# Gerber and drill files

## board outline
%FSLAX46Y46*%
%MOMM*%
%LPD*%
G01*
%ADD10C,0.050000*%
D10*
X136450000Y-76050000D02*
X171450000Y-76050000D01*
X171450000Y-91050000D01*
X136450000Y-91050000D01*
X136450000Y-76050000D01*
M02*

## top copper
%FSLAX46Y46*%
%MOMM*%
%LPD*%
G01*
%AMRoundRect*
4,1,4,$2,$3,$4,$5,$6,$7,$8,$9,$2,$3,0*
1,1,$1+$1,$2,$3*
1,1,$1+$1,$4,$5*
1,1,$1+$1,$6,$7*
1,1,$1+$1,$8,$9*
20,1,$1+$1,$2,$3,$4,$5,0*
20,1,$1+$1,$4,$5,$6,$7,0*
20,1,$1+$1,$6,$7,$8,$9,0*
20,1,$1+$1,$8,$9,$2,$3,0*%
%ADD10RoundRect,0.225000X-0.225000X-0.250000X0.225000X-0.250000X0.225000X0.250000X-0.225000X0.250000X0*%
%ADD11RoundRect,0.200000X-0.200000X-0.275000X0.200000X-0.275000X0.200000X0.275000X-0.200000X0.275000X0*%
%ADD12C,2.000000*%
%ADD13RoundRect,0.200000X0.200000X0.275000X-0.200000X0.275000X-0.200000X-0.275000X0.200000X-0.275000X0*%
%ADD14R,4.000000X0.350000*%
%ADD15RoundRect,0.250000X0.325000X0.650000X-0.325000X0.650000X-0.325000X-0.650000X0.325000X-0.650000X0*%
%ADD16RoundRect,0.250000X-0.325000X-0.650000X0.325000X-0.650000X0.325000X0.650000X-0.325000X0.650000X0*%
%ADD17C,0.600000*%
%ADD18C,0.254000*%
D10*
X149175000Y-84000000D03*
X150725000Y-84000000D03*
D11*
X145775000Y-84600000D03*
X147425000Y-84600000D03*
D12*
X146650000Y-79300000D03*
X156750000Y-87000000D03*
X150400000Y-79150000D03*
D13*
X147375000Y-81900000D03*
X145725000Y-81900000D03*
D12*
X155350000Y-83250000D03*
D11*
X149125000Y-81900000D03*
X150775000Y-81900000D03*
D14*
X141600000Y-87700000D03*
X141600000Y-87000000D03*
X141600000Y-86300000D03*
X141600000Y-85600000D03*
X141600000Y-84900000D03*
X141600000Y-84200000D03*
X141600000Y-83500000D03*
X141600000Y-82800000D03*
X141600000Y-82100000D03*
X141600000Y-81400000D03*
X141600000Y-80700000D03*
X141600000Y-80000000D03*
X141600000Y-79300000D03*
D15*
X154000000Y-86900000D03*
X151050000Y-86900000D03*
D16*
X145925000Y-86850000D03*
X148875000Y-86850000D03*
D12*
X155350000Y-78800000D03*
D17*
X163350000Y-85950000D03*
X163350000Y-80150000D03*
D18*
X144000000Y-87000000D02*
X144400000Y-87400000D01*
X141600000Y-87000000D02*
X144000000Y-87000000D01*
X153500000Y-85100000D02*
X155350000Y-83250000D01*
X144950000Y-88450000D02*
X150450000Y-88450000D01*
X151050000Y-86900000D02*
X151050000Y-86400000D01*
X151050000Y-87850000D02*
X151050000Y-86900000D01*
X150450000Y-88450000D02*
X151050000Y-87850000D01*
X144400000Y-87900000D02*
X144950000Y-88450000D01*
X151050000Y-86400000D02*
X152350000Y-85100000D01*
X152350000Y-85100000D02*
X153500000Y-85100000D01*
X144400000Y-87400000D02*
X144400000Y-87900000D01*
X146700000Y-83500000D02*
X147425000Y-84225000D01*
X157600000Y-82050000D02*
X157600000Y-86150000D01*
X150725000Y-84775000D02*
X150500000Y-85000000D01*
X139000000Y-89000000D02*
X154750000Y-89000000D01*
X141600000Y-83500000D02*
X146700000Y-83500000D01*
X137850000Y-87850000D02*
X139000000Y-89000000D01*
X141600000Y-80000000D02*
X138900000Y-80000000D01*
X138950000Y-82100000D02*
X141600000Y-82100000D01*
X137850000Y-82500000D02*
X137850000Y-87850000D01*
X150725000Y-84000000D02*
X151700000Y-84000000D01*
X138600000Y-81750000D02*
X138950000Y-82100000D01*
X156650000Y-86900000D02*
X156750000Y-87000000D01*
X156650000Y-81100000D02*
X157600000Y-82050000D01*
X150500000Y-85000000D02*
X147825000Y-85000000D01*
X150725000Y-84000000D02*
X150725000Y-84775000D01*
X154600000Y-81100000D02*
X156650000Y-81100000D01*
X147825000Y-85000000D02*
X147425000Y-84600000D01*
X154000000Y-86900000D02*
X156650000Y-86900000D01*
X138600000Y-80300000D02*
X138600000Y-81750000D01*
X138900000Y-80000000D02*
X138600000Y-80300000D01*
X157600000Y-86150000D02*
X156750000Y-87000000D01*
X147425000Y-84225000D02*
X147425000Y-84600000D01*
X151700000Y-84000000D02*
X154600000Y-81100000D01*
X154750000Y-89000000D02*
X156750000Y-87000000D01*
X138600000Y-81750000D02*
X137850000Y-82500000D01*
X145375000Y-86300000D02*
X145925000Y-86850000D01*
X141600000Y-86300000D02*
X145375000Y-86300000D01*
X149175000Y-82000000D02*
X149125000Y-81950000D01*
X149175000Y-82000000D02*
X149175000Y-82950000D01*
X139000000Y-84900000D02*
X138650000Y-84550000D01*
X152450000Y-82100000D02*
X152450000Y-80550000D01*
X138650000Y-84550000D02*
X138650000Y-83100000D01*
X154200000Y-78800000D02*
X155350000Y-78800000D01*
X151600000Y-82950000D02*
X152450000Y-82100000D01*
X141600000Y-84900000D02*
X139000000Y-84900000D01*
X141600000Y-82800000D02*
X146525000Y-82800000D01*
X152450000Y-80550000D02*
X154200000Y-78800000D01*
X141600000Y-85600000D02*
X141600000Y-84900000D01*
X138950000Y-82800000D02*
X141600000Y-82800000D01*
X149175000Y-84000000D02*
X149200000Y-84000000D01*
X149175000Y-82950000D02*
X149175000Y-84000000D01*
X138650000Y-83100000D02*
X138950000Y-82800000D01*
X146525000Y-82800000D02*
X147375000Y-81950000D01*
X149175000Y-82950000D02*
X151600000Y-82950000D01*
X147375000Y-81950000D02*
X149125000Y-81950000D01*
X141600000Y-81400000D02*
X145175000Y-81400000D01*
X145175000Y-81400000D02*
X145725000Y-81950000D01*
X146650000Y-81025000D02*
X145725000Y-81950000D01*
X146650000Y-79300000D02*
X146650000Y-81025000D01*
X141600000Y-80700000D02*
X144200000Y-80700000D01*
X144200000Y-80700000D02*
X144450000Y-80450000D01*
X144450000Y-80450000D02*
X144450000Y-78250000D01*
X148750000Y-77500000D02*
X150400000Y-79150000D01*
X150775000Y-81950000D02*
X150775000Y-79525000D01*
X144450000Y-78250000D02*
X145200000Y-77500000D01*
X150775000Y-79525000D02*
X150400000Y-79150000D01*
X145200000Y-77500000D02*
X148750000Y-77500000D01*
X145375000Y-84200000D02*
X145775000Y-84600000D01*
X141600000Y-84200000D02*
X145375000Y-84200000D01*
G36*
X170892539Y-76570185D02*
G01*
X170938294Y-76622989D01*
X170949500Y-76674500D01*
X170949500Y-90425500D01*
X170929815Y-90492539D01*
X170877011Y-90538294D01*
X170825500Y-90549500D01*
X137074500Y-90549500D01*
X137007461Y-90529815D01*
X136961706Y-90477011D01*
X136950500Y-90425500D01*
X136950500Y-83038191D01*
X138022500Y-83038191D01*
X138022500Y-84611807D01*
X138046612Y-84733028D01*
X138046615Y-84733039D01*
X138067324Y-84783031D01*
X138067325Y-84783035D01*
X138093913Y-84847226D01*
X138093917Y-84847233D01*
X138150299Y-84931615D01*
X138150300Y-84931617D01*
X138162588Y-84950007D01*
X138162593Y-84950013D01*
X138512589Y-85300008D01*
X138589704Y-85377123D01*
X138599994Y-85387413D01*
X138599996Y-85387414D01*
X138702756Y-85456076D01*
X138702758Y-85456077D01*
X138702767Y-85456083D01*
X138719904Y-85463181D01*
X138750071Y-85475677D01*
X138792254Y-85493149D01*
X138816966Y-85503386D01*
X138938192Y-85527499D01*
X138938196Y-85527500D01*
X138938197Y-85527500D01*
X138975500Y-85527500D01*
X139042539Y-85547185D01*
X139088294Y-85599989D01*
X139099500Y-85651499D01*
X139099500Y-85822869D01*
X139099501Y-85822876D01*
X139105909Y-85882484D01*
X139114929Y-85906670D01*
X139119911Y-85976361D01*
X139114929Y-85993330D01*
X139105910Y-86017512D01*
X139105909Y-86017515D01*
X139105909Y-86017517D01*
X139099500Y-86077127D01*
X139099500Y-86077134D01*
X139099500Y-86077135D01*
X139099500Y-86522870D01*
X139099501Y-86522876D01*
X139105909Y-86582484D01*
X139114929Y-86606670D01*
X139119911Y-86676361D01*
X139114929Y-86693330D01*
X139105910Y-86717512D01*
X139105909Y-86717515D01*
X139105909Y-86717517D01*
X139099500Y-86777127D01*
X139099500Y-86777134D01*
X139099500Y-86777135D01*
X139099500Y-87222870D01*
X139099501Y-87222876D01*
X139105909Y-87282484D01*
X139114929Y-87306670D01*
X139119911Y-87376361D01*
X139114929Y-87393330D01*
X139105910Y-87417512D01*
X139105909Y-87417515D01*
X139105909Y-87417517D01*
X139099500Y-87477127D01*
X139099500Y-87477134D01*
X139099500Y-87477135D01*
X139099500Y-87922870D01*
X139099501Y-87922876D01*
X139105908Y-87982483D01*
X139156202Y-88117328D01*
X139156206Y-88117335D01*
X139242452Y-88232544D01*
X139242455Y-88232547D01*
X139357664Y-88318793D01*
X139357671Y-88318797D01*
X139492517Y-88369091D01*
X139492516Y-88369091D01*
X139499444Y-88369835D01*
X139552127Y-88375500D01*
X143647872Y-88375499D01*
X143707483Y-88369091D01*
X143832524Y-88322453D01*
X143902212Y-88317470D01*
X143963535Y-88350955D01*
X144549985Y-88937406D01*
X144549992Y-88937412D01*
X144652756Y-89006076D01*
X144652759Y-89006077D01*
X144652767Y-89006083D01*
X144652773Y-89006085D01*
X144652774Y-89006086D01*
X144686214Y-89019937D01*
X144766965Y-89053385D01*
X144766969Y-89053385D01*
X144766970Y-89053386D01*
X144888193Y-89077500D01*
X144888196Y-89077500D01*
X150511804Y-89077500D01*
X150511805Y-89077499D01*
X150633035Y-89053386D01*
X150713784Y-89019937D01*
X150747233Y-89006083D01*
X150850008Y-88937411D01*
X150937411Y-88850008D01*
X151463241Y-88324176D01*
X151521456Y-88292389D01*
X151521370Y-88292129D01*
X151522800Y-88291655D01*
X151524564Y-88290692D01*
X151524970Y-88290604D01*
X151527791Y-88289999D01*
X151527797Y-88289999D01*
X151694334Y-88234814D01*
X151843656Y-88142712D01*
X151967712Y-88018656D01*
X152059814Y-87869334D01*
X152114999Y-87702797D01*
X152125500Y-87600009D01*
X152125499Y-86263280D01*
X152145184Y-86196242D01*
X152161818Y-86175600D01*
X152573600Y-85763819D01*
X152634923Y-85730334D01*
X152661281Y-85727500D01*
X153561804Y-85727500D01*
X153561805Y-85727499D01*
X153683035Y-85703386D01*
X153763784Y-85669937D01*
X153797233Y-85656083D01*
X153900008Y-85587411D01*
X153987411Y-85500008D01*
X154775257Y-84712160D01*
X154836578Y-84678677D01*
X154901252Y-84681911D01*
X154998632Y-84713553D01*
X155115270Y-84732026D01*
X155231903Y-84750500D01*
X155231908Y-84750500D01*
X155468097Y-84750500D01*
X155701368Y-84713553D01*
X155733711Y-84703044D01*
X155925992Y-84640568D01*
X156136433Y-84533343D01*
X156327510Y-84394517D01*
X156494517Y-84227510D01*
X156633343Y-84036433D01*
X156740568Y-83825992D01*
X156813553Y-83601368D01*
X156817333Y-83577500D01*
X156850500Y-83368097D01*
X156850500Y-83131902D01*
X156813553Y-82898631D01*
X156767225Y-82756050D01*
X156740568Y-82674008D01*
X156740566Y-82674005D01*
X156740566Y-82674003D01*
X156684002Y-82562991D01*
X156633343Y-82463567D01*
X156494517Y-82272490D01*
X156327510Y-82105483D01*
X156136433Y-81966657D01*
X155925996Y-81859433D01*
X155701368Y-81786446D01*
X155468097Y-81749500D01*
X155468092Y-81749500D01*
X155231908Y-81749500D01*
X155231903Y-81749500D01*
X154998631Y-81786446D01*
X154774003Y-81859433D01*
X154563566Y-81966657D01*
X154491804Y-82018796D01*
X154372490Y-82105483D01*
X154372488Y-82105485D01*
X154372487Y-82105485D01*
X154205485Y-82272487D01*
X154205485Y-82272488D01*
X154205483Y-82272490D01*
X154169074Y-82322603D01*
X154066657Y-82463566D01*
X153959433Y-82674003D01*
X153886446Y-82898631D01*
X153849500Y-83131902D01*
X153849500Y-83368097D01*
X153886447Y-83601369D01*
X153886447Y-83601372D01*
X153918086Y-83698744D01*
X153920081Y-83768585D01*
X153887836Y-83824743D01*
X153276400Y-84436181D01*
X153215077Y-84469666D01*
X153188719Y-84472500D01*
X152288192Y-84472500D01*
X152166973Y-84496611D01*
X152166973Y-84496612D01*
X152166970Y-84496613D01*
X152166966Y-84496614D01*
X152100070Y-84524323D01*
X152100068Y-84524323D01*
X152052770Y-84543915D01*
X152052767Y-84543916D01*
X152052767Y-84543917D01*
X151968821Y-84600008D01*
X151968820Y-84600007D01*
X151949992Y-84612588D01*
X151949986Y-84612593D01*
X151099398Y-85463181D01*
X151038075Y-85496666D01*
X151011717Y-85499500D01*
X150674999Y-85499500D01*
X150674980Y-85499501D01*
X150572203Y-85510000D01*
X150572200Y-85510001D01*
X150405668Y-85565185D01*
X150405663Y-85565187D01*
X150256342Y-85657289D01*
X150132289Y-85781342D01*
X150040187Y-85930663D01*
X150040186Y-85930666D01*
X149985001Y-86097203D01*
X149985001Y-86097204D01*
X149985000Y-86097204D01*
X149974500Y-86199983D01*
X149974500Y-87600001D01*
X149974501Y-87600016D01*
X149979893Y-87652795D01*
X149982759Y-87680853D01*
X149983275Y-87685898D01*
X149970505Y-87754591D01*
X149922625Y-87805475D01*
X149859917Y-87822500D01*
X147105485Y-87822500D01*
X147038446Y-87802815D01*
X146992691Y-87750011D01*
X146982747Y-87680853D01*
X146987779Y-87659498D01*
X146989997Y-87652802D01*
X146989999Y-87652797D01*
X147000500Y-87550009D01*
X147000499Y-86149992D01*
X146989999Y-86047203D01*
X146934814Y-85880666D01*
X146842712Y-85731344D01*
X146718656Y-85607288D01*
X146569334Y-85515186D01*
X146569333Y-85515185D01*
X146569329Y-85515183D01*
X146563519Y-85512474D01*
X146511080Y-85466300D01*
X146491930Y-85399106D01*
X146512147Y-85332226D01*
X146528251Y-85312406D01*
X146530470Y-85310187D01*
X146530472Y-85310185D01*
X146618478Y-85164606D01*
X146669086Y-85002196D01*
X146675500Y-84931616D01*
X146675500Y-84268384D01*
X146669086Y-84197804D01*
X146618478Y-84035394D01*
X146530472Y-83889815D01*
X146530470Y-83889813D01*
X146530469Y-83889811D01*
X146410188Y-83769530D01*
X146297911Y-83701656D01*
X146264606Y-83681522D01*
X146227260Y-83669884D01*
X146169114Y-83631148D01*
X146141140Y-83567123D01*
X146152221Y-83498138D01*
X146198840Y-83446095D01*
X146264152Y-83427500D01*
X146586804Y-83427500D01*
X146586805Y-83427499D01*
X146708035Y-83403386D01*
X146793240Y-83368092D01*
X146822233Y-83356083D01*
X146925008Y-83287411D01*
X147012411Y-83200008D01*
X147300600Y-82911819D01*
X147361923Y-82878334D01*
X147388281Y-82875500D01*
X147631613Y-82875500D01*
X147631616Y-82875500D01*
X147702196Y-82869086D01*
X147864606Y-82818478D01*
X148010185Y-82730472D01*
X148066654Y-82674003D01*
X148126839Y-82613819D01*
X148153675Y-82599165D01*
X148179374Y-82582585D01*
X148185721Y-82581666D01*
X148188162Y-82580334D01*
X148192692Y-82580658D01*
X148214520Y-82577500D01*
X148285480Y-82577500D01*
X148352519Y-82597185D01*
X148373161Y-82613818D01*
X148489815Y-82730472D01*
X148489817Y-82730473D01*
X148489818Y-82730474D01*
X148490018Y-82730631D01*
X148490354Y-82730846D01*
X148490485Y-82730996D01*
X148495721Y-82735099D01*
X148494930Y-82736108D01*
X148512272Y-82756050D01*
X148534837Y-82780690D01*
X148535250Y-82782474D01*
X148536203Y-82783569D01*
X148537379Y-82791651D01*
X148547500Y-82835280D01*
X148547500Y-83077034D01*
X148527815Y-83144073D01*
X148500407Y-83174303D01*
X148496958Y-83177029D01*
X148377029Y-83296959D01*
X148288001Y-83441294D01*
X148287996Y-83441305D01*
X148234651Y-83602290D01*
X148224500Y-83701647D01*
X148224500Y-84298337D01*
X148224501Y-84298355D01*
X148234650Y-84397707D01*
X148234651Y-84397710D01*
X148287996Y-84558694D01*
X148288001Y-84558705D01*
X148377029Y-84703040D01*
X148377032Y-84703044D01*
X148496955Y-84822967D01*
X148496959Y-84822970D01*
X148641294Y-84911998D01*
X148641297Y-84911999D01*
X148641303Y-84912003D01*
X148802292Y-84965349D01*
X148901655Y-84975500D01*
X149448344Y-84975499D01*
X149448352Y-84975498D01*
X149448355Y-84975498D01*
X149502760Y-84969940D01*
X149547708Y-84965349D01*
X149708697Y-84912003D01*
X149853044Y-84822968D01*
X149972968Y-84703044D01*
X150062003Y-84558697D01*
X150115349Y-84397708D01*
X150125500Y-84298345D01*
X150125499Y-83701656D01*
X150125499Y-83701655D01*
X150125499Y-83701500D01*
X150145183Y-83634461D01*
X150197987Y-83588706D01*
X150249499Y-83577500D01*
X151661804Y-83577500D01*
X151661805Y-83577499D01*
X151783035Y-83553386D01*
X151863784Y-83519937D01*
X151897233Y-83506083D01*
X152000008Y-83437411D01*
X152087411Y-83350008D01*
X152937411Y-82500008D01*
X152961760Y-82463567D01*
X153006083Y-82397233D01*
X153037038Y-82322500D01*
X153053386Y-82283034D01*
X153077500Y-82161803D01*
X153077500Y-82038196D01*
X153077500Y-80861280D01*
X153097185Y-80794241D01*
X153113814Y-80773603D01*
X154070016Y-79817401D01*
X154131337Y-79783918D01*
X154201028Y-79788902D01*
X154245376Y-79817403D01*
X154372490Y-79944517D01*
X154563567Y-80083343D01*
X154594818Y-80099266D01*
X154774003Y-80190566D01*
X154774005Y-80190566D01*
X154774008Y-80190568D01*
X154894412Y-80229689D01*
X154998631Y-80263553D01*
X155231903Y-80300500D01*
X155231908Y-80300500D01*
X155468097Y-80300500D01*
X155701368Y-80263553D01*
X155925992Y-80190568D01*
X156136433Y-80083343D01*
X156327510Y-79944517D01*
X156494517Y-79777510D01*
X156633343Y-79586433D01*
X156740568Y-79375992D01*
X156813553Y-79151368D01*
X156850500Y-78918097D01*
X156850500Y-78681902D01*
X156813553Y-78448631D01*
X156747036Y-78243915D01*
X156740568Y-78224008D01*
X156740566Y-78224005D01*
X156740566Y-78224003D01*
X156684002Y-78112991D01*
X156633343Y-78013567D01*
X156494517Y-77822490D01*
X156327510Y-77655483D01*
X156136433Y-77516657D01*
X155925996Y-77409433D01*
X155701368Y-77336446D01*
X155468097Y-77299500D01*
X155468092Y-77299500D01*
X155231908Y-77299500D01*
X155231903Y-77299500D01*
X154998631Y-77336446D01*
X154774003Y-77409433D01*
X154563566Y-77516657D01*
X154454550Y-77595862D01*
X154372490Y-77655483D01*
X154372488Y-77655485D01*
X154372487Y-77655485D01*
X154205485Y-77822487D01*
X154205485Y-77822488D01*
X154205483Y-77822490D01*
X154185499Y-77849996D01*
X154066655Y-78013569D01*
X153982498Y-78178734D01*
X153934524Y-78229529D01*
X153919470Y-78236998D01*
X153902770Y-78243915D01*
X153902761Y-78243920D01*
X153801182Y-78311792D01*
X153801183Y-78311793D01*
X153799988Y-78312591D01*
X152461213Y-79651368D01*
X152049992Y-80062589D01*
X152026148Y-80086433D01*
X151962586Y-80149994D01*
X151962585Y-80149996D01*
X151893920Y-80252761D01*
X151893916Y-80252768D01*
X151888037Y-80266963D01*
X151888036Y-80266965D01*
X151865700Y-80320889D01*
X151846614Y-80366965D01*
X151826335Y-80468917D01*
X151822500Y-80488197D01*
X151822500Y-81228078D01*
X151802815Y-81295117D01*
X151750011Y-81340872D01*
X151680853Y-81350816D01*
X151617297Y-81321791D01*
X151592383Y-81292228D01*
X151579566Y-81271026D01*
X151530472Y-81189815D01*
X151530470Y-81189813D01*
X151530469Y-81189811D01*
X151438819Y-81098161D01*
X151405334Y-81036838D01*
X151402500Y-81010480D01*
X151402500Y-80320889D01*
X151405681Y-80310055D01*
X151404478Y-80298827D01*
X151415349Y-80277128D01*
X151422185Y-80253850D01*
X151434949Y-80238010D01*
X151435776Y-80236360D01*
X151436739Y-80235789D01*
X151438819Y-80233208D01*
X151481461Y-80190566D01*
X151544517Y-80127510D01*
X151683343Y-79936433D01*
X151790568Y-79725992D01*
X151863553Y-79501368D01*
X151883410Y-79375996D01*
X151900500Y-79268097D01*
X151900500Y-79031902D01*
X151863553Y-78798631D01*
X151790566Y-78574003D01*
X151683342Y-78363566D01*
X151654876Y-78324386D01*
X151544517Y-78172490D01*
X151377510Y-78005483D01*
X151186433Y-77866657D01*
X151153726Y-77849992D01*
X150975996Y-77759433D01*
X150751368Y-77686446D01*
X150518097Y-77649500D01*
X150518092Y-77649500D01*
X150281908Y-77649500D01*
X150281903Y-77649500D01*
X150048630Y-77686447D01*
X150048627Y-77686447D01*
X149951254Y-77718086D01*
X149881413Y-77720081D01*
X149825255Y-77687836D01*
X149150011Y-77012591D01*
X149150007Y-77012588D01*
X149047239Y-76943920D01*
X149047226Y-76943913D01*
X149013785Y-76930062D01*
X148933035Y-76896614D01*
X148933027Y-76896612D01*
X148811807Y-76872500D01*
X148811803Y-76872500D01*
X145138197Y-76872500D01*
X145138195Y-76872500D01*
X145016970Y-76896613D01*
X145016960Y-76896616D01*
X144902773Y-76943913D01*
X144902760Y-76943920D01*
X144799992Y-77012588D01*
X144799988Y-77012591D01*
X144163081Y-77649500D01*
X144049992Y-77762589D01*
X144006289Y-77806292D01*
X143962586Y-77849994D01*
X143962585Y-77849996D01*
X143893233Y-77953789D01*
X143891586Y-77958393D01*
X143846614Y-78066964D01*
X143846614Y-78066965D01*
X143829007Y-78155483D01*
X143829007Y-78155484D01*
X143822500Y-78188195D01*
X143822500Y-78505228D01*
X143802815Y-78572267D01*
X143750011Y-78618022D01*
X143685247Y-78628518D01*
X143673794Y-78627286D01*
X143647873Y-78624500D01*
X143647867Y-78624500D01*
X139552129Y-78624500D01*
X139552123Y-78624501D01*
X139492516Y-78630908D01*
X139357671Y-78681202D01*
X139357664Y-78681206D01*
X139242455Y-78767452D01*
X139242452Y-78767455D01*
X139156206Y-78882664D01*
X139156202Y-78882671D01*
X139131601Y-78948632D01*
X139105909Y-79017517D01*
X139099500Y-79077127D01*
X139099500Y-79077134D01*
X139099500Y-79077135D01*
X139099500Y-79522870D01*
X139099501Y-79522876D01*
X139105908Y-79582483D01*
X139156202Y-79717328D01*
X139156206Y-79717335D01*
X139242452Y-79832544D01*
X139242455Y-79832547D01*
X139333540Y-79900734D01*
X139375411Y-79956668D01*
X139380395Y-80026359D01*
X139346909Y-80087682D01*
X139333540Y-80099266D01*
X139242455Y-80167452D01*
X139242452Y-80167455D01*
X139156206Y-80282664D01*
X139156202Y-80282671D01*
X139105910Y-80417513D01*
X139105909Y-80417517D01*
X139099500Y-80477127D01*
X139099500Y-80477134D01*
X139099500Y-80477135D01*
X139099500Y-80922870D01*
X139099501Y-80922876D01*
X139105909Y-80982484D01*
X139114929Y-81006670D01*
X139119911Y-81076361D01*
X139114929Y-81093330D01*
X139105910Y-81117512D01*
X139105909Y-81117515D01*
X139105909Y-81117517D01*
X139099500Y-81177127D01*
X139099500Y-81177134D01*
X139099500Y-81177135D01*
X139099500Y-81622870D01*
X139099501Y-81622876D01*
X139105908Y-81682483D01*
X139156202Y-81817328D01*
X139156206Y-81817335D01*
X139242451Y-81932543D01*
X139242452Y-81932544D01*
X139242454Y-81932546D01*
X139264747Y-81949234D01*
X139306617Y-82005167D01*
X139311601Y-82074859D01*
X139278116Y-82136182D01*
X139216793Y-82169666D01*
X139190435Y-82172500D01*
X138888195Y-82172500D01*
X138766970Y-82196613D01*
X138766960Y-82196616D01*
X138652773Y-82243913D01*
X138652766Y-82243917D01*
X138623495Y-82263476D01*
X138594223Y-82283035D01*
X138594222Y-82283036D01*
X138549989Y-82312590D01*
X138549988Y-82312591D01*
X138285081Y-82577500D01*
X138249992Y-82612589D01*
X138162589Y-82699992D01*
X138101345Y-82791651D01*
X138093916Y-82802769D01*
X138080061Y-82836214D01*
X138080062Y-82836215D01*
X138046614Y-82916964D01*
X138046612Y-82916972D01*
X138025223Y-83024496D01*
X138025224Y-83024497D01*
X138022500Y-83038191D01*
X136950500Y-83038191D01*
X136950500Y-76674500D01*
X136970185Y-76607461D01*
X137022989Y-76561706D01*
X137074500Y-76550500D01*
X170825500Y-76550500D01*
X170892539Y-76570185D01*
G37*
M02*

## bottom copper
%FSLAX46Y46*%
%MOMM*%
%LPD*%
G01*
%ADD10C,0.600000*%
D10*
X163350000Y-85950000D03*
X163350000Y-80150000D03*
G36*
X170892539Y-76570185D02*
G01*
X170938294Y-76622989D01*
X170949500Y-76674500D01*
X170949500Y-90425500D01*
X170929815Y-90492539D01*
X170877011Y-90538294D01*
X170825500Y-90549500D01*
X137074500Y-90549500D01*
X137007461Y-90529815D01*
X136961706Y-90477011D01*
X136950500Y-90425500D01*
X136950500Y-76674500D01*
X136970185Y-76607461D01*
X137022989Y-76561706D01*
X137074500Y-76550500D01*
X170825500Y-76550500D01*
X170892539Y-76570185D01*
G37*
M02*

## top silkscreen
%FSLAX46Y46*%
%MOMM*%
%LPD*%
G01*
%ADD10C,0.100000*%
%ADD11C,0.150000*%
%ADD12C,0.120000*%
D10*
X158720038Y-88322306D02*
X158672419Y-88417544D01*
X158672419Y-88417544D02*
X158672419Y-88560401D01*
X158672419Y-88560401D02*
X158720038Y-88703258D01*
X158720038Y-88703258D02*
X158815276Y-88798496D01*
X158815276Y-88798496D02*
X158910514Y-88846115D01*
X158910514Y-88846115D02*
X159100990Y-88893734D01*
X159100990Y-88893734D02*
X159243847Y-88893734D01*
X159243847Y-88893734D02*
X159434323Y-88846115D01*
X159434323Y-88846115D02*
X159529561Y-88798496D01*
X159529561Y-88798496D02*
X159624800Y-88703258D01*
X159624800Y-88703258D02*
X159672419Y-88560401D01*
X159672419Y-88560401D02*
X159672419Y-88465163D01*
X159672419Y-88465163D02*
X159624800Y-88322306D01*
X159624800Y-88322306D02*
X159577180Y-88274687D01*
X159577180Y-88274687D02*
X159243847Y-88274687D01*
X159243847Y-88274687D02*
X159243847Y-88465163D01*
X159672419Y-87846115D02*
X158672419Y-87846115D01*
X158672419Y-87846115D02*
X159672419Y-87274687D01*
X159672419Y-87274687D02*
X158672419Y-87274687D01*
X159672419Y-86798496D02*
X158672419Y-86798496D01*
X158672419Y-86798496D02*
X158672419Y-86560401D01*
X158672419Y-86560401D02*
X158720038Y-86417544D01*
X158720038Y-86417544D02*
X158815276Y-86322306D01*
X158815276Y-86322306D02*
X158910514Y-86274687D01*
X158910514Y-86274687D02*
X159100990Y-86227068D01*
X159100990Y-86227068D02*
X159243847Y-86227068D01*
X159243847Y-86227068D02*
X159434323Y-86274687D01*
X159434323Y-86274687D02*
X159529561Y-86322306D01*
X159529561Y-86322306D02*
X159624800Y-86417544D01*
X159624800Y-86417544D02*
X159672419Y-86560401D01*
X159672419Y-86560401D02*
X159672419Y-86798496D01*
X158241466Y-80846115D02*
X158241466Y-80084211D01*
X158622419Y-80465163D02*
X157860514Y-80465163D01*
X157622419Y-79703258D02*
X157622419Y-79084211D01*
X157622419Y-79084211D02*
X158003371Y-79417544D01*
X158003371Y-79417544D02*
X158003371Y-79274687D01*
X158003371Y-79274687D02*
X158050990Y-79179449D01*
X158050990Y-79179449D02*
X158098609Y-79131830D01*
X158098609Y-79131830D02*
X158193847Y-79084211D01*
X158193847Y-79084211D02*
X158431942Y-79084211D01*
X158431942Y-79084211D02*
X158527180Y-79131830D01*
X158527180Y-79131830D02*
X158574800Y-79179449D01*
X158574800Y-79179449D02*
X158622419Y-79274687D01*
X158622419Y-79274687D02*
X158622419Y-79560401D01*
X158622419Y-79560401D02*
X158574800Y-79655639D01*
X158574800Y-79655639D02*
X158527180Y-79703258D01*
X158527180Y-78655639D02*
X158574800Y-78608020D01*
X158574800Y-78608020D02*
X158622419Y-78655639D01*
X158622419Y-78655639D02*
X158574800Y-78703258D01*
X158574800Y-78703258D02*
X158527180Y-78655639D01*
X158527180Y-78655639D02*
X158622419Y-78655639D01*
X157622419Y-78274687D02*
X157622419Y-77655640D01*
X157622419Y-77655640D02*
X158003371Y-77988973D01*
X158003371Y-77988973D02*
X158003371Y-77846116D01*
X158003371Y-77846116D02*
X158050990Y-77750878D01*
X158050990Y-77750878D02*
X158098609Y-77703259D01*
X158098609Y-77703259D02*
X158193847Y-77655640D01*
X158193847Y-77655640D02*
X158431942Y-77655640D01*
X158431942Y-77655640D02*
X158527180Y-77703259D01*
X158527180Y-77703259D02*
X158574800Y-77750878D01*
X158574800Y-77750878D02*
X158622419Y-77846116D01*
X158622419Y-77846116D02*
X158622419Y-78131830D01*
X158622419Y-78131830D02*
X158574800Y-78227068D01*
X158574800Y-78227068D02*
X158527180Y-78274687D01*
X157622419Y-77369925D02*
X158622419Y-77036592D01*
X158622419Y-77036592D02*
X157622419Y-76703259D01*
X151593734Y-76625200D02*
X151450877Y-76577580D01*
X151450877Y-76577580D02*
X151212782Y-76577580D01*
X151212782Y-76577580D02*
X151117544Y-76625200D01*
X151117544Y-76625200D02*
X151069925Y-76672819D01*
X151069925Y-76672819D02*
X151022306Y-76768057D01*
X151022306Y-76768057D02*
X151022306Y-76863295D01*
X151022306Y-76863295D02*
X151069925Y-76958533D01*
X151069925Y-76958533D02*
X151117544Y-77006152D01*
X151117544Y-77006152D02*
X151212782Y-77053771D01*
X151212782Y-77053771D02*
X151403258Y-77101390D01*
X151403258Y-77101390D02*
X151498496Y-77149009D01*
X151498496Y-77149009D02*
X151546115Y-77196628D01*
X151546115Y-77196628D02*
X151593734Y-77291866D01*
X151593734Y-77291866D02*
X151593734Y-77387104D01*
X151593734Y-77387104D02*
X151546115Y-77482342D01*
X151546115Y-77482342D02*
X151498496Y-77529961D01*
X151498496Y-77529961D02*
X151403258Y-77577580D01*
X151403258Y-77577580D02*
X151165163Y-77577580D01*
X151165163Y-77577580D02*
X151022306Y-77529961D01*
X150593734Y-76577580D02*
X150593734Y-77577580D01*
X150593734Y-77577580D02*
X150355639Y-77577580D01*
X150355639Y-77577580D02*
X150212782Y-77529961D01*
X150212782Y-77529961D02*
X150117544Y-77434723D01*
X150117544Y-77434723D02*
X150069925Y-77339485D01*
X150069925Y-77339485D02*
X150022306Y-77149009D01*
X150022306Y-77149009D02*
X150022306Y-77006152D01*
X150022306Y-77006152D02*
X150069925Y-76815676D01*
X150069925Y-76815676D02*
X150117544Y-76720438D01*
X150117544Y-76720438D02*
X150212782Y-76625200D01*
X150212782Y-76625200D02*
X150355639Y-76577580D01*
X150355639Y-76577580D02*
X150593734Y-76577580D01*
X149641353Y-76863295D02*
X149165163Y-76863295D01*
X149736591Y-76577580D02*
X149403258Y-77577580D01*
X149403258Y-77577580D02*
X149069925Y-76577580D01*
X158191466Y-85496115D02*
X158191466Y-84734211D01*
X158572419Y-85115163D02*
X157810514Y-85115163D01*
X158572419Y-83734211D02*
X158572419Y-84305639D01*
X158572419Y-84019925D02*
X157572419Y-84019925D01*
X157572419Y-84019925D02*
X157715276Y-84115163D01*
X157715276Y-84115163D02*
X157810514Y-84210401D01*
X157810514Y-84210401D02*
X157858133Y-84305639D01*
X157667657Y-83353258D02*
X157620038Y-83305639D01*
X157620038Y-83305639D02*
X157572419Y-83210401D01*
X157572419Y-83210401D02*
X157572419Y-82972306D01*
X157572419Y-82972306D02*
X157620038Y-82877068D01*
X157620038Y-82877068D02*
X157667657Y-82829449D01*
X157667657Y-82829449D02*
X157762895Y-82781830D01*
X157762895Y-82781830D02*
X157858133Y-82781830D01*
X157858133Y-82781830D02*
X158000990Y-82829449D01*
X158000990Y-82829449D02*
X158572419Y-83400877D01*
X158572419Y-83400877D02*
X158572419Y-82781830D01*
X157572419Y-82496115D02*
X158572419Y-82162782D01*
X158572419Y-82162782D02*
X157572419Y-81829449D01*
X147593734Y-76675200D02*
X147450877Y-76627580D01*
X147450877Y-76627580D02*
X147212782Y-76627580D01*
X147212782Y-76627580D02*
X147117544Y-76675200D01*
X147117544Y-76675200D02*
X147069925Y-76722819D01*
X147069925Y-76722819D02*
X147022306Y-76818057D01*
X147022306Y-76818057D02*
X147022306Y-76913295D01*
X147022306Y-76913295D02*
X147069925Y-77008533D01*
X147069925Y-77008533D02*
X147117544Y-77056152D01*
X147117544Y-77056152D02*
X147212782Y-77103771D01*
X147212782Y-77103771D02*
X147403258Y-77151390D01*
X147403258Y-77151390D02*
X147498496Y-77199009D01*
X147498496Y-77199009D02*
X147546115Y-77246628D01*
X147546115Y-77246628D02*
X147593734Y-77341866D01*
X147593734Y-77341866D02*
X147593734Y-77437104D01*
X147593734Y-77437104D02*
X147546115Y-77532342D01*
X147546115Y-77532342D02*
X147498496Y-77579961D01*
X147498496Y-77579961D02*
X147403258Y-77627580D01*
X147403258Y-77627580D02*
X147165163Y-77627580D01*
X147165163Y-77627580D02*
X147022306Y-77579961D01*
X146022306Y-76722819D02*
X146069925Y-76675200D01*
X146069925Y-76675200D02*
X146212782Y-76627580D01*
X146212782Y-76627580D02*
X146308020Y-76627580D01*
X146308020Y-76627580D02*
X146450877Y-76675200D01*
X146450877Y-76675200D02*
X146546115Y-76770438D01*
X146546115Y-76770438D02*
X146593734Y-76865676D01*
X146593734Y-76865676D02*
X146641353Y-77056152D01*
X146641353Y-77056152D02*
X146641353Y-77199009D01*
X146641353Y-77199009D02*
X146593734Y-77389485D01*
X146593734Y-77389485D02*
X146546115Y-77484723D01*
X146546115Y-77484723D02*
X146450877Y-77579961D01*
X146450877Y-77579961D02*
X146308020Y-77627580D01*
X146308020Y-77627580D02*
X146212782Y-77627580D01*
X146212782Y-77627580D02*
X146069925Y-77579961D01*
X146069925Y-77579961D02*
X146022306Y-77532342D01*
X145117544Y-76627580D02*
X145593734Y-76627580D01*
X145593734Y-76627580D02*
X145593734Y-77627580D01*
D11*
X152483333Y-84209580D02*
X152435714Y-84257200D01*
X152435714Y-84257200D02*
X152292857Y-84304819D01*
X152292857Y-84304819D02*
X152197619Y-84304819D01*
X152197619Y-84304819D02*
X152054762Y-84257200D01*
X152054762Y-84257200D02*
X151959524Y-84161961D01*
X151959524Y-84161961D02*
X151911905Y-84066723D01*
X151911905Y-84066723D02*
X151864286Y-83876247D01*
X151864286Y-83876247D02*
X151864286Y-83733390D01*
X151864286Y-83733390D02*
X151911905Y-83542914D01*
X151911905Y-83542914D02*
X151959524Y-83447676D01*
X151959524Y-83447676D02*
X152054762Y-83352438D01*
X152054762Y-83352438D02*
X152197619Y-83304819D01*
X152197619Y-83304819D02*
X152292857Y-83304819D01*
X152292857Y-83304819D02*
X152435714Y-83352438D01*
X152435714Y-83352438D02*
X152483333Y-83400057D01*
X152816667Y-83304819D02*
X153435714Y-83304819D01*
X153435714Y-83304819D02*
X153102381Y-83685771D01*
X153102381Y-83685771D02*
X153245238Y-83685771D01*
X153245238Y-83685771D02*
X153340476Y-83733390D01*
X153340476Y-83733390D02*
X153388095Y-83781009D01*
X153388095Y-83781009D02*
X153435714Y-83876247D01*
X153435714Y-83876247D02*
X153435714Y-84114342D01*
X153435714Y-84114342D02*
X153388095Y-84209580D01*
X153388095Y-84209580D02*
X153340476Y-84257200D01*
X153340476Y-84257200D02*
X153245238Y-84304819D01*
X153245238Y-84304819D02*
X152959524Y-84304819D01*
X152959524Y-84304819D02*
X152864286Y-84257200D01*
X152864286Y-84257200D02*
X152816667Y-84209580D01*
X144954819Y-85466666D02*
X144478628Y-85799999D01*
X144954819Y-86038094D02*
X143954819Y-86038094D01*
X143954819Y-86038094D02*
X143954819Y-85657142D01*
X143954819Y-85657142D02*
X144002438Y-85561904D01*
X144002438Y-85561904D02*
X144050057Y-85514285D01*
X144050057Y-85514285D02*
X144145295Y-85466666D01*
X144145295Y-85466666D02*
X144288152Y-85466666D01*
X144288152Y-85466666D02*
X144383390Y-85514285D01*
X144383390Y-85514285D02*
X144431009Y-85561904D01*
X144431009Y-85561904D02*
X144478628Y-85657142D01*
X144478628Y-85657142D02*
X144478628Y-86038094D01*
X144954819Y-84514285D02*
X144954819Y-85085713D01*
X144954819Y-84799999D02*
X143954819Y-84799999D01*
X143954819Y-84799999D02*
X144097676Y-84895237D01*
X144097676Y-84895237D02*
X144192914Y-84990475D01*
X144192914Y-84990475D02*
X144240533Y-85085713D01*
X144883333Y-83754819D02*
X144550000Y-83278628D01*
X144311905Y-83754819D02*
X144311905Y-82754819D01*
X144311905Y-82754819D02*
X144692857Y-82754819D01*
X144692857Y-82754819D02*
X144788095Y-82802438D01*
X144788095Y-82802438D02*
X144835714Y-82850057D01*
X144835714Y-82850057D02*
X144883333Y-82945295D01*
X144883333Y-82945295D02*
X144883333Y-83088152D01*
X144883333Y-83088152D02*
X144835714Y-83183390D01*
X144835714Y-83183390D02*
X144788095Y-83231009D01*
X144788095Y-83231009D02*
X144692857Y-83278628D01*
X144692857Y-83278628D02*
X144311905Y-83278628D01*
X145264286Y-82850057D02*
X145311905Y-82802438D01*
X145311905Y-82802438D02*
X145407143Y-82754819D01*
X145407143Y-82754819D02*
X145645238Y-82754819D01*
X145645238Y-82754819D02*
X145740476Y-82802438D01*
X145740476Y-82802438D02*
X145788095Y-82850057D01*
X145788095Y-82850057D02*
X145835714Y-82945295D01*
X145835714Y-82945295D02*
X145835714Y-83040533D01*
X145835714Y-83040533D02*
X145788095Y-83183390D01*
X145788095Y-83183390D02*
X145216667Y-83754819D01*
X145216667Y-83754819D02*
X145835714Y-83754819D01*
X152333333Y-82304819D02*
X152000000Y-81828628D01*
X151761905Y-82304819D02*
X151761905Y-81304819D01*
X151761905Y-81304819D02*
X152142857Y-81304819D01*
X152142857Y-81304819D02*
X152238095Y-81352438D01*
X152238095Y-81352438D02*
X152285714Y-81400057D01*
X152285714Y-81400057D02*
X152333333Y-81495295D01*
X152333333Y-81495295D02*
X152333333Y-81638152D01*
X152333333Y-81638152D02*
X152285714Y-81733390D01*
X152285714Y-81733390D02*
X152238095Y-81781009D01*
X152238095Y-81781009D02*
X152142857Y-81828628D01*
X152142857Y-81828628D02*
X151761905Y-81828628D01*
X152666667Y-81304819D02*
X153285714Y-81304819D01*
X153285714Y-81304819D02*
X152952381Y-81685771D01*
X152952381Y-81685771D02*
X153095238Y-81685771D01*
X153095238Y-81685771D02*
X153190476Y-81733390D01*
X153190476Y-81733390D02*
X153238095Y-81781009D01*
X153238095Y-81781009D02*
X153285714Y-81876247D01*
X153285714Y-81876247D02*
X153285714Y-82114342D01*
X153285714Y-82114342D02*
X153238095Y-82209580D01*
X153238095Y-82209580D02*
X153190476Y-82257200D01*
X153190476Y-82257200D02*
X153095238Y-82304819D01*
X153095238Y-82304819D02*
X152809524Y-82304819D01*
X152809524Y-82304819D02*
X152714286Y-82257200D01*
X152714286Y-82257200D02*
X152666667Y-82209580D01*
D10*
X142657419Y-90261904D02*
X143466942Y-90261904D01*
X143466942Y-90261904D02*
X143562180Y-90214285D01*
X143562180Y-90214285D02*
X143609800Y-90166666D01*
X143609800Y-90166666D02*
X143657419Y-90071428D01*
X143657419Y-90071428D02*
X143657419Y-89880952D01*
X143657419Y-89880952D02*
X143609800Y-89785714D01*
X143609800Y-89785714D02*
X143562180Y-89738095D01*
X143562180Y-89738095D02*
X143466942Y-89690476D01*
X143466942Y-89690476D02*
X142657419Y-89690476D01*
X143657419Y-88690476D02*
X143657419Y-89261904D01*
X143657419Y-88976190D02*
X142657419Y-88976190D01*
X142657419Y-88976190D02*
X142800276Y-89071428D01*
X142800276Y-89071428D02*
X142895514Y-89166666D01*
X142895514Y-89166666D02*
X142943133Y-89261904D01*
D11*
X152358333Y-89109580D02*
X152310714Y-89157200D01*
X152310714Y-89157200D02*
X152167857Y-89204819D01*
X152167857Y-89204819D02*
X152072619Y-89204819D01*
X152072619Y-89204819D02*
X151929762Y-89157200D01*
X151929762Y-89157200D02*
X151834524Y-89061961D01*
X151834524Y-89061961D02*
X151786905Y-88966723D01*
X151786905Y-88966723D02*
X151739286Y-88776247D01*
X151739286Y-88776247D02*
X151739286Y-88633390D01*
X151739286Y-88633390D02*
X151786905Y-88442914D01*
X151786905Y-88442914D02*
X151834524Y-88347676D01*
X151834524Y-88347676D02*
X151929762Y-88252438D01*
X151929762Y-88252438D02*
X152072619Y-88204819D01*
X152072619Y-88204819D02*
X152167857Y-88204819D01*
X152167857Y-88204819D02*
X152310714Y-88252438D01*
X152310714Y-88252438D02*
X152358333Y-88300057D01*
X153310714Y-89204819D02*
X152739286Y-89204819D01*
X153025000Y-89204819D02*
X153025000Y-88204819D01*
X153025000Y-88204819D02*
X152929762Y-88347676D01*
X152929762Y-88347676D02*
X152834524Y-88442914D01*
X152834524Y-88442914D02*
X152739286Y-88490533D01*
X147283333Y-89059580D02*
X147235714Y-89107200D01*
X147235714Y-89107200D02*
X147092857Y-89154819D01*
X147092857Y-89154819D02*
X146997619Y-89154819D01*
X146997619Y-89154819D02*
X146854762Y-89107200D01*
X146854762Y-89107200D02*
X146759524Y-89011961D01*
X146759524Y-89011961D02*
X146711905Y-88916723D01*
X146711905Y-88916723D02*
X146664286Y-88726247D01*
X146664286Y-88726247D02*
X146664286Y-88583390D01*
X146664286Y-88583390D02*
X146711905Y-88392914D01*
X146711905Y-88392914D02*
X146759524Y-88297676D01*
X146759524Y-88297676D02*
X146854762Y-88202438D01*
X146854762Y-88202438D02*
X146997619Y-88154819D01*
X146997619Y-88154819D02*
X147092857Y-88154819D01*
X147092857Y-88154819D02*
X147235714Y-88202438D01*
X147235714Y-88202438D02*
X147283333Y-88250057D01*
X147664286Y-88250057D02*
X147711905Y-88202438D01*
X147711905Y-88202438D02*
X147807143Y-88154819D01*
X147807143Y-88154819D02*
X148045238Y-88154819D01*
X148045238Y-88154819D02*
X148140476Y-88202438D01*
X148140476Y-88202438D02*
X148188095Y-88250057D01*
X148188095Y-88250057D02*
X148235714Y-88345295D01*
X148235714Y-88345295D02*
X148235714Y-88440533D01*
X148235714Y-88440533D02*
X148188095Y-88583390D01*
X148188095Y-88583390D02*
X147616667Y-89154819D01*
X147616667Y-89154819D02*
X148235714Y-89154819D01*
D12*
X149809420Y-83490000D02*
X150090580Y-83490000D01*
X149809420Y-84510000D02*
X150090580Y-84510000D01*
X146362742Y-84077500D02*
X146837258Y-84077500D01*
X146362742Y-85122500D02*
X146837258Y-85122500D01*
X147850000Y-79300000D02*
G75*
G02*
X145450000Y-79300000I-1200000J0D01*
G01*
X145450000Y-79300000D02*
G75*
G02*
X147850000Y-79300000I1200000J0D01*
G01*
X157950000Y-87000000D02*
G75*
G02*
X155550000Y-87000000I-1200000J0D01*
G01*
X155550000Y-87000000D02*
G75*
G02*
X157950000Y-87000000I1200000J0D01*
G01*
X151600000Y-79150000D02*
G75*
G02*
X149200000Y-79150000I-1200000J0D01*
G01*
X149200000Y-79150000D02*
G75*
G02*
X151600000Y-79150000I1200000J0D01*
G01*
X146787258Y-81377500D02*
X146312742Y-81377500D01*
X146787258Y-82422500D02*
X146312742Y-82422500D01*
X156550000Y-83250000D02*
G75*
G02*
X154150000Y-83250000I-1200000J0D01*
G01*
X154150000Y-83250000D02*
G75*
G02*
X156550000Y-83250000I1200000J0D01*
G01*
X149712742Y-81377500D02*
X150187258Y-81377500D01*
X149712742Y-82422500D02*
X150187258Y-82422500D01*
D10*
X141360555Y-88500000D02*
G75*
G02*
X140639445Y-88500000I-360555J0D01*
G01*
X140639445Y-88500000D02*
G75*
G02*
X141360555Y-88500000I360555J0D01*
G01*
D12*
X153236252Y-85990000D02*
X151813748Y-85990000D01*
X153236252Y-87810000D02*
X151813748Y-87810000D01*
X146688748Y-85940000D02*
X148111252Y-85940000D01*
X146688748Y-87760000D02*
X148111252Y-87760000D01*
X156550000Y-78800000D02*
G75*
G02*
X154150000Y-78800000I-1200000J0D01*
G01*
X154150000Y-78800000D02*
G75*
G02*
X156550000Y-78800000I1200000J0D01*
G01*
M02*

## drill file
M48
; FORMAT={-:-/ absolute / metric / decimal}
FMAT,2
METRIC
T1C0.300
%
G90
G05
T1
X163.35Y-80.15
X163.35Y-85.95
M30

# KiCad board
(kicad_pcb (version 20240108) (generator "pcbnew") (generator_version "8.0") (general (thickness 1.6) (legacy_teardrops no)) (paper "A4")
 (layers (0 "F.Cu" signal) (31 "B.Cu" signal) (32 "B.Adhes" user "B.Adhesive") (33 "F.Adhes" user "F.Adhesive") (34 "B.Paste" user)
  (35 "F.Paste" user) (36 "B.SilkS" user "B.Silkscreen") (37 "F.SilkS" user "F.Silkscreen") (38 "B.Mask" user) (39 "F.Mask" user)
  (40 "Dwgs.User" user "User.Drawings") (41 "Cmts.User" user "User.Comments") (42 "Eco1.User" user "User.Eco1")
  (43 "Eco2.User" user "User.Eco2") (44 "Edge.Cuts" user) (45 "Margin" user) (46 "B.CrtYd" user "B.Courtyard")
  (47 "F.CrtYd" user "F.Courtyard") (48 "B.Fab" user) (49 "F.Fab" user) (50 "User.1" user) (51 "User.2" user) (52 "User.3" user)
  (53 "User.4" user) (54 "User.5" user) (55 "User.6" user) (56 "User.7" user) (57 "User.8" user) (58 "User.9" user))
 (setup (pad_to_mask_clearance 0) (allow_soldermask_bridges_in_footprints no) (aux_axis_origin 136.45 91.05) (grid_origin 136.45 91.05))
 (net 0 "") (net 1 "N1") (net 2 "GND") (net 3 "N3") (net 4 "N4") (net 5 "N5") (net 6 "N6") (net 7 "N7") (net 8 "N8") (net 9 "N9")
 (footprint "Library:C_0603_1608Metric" (layer "F.Cu") (at 149.95 84)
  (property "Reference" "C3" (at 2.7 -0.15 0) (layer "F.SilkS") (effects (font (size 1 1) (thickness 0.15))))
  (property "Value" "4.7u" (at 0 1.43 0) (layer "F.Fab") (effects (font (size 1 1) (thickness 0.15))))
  (fp_line (start -0.14058 -0.51) (end 0.14058 -0.51) (stroke (width 0.12) (type solid)) (layer "F.SilkS"))
  (fp_line (start -0.14058 0.51) (end 0.14058 0.51) (stroke (width 0.12) (type solid)) (layer "F.SilkS"))
  (pad "1" smd roundrect (at -0.775 0) (size 0.9 0.95) (layers "F.Cu" "F.Paste" "F.Mask") (roundrect_rratio 0.25) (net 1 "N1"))
  (pad "2" smd roundrect (at 0.775 0) (size 0.9 0.95) (layers "F.Cu" "F.Paste" "F.Mask") (roundrect_rratio 0.25) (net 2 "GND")))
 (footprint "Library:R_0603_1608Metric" (layer "F.Cu") (at 146.6 84.6)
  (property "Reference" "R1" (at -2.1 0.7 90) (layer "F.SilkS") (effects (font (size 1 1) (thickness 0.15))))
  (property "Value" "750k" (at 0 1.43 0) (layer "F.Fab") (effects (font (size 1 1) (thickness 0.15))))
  (fp_line (start -0.237258 -0.5225) (end 0.237258 -0.5225) (stroke (width 0.12) (type solid)) (layer "F.SilkS"))
  (fp_line (start -0.237258 0.5225) (end 0.237258 0.5225) (stroke (width 0.12) (type solid)) (layer "F.SilkS"))
  (pad "1" smd roundrect (at -0.825 0) (size 0.8 0.95) (layers "F.Cu" "F.Paste" "F.Mask") (roundrect_rratio 0.25) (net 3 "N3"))
  (pad "2" smd roundrect (at 0.825 0) (size 0.8 0.95) (layers "F.Cu" "F.Paste" "F.Mask") (roundrect_rratio 0.25) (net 2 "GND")))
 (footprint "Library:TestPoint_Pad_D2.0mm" (layer "F.Cu") (at 146.65 79.3)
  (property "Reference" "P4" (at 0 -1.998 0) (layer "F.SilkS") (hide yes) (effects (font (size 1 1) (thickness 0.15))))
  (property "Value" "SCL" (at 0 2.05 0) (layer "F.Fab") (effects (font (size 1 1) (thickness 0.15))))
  (fp_circle (center 0 0) (end 0 1.2) (stroke (width 0.12) (type solid)) (fill none) (layer "F.SilkS"))
  (pad "1" smd circle (at 0 0) (size 2 2) (layers "F.Cu" "F.Mask") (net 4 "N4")))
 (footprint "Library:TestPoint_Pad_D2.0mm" (layer "F.Cu") (at 156.75 87)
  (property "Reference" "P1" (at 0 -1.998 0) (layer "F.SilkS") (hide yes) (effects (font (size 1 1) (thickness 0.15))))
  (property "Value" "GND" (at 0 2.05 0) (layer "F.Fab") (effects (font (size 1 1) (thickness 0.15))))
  (fp_circle (center 0 0) (end 0 1.2) (stroke (width 0.12) (type solid)) (fill none) (layer "F.SilkS"))
  (pad "1" smd circle (at 0 0) (size 2 2) (layers "F.Cu" "F.Mask") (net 2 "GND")))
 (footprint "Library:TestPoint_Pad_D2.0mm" (layer "F.Cu") (at 150.4 79.15)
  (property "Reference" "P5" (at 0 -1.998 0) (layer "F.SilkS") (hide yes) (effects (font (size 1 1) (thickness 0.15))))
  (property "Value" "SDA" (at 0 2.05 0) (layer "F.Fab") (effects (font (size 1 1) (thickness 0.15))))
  (fp_circle (center 0 0) (end 0 1.2) (stroke (width 0.12) (type solid)) (fill none) (layer "F.SilkS"))
  (pad "1" smd circle (at 0 0) (size 2 2) (layers "F.Cu" "F.Mask") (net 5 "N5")))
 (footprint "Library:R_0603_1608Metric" (layer "F.Cu") (at 146.55 81.9 180)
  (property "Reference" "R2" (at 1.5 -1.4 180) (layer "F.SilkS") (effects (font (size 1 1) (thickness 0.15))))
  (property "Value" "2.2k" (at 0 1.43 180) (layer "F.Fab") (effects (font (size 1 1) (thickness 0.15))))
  (fp_line (start -0.237258 0.5225) (end 0.237258 0.5225) (stroke (width 0.12) (type solid)) (layer "F.SilkS"))
  (fp_line (start -0.237258 -0.5225) (end 0.237258 -0.5225) (stroke (width 0.12) (type solid)) (layer "F.SilkS"))
  (pad "1" smd roundrect (at -0.825 0 180) (size 0.8 0.95) (layers "F.Cu" "F.Paste" "F.Mask") (roundrect_rratio 0.25) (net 1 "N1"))
  (pad "2" smd roundrect (at 0.825 0 180) (size 0.8 0.95) (layers "F.Cu" "F.Paste" "F.Mask") (roundrect_rratio 0.25) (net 4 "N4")))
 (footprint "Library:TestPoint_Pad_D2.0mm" (layer "F.Cu") (at 155.35 83.25)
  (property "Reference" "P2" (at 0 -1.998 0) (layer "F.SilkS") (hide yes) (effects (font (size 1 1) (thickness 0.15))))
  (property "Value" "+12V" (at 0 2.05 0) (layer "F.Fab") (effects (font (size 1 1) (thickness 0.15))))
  (fp_circle (center 0 0) (end 0 1.2) (stroke (width 0.12) (type solid)) (fill none) (layer "F.SilkS"))
  (pad "1" smd circle (at 0 0) (size 2 2) (layers "F.Cu" "F.Mask") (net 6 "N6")))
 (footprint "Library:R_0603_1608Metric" (layer "F.Cu") (at 149.95 81.9)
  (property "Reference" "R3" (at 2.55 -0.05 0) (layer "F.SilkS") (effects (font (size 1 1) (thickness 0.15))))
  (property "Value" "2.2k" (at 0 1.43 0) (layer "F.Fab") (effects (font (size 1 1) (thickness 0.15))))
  (fp_line (start -0.237258 -0.5225) (end 0.237258 -0.5225) (stroke (width 0.12) (type solid)) (layer "F.SilkS"))
  (fp_line (start -0.237258 0.5225) (end 0.237258 0.5225) (stroke (width 0.12) (type solid)) (layer "F.SilkS"))
  (pad "1" smd roundrect (at -0.825 0) (size 0.8 0.95) (layers "F.Cu" "F.Paste" "F.Mask") (roundrect_rratio 0.25) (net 1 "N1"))
  (pad "2" smd roundrect (at 0.825 0) (size 0.8 0.95) (layers "F.Cu" "F.Paste" "F.Mask") (roundrect_rratio 0.25) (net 5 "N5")))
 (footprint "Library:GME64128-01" (layer "F.Cu") (at 141.6 83.5 90)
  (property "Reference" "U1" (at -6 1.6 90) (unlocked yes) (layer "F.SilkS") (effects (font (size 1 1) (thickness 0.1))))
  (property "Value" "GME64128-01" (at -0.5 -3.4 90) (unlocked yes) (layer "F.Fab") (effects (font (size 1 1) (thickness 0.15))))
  (fp_circle (center -5 -0.6) (end -4.7 -0.4) (stroke (width 0.1) (type default)) (fill none) (layer "F.SilkS"))
  (pad "1" smd rect (at -4.2 0 90) (size 0.35 4) (layers "F.Cu" "F.Paste" "F.Mask") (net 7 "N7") (thermal_bridge_angle 45))
  (pad "2" smd rect (at -3.5 0 90) (size 0.35 4) (layers "F.Cu" "F.Paste" "F.Mask") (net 6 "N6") (thermal_bridge_angle 45))
  (pad "3" smd rect (at -2.8 0 90) (size 0.35 4) (layers "F.Cu" "F.Paste" "F.Mask") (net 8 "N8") (thermal_bridge_angle 45))
  (pad "4" smd rect (at -2.1 0 90) (size 0.35 4) (layers "F.Cu" "F.Paste" "F.Mask") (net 1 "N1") (thermal_bridge_angle 45))
  (pad "5" smd rect (at -1.4 0 90) (size 0.35 4) (layers "F.Cu" "F.Paste" "F.Mask") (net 1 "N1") (thermal_bridge_angle 45))
  (pad "6" smd rect (at -0.7 0 90) (size 0.35 4) (layers "F.Cu" "F.Paste" "F.Mask") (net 3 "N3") (thermal_bridge_angle 45))
  (pad "7" smd rect (at 0 0 90) (size 0.35 4) (layers "F.Cu" "F.Paste" "F.Mask") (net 2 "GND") (thermal_bridge_angle 45))
  (pad "8" smd rect (at 0.7 0 90) (size 0.35 4) (layers "F.Cu" "F.Paste" "F.Mask") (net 1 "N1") (thermal_bridge_angle 45))
  (pad "9" smd rect (at 1.4 0 90) (size 0.35 4) (layers "F.Cu" "F.Paste" "F.Mask") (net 2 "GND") (thermal_bridge_angle 45))
  (pad "10" smd rect (at 2.1 0 90) (size 0.35 4) (layers "F.Cu" "F.Paste" "F.Mask") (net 4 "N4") (thermal_bridge_angle 45))
  (pad "11" smd rect (at 2.8 0 90) (size 0.35 4) (layers "F.Cu" "F.Paste" "F.Mask") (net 5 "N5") (thermal_bridge_angle 45))
  (pad "12" smd rect (at 3.5 0 90) (size 0.35 4) (layers "F.Cu" "F.Paste" "F.Mask") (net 2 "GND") (thermal_bridge_angle 45))
  (pad "13" smd rect (at 4.2 0 90) (size 0.35 4) (layers "F.Cu" "F.Paste" "F.Mask") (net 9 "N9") (thermal_bridge_angle 45)))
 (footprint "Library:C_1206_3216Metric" (layer "F.Cu") (at 152.525 86.9 180)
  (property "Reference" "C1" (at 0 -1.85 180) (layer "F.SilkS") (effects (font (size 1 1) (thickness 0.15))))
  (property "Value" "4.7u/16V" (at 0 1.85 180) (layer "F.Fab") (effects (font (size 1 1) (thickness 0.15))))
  (fp_line (start -0.711252 0.91) (end 0.711252 0.91) (stroke (width 0.12) (type solid)) (layer "F.SilkS"))
  (fp_line (start -0.711252 -0.91) (end 0.711252 -0.91) (stroke (width 0.12) (type solid)) (layer "F.SilkS"))
  (pad "1" smd roundrect (at -1.475 0 180) (size 1.15 1.8) (layers "F.Cu" "F.Paste" "F.Mask") (roundrect_rratio 0.217391) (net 2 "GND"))
  (pad "2" smd roundrect (at 1.475 0 180) (size 1.15 1.8) (layers "F.Cu" "F.Paste" "F.Mask") (roundrect_rratio 0.217391) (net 6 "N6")))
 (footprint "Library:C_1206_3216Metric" (layer "F.Cu") (at 147.4 86.85)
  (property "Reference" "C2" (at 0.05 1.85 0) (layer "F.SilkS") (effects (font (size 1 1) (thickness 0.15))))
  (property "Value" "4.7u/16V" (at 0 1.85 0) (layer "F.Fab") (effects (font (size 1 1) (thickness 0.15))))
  (fp_line (start -0.711252 -0.91) (end 0.711252 -0.91) (stroke (width 0.12) (type solid)) (layer "F.SilkS"))
  (fp_line (start -0.711252 0.91) (end 0.711252 0.91) (stroke (width 0.12) (type solid)) (layer "F.SilkS"))
  (pad "1" smd roundrect (at -1.475 0) (size 1.15 1.8) (layers "F.Cu" "F.Paste" "F.Mask") (roundrect_rratio 0.217391) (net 8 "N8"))
  (pad "2" smd roundrect (at 1.475 0) (size 1.15 1.8) (layers "F.Cu" "F.Paste" "F.Mask") (roundrect_rratio 0.217391) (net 2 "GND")))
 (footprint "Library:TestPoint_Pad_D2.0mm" (layer "F.Cu") (at 155.35 78.8)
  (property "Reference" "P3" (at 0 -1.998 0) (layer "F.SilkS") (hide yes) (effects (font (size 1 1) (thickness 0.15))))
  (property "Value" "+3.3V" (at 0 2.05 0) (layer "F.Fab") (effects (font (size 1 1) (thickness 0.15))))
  (fp_circle (center 0 0) (end 0 1.2) (stroke (width 0.12) (type solid)) (fill none) (layer "F.SilkS"))
  (pad "1" smd circle (at 0 0) (size 2 2) (layers "F.Cu" "F.Mask") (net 1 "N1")))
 (gr_rect (start 136.45 76.05) (end 171.45 91.05) (stroke (width 0.05) (type default)) (fill none) (layer "Edge.Cuts"))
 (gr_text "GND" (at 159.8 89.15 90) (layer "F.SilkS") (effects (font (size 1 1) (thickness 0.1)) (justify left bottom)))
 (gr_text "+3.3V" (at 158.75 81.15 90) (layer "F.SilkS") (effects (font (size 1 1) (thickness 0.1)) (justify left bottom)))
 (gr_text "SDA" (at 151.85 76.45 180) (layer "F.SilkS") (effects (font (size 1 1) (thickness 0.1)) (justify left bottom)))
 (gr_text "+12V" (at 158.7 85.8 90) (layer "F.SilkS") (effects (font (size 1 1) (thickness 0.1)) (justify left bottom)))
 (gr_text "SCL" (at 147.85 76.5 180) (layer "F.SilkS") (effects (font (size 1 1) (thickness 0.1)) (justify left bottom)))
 (segment (start 144 87) (end 144.4 87.4) (width 0.254) (layer "F.Cu") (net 6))
 (segment (start 141.6 87) (end 144 87) (width 0.254) (layer "F.Cu") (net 6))
 (segment (start 153.5 85.1) (end 155.35 83.25) (width 0.254) (layer "F.Cu") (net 6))
 (segment (start 144.95 88.45) (end 150.45 88.45) (width 0.254) (layer "F.Cu") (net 6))
 (segment (start 151.05 86.9) (end 151.05 86.4) (width 0.254) (layer "F.Cu") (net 6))
 (segment (start 151.05 87.85) (end 151.05 86.9) (width 0.254) (layer "F.Cu") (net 6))
 (segment (start 150.45 88.45) (end 151.05 87.85) (width 0.254) (layer "F.Cu") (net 6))
 (segment (start 144.4 87.9) (end 144.95 88.45) (width 0.254) (layer "F.Cu") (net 6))
 (segment (start 151.05 86.4) (end 152.35 85.1) (width 0.254) (layer "F.Cu") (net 6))
 (segment (start 152.35 85.1) (end 153.5 85.1) (width 0.254) (layer "F.Cu") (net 6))
 (segment (start 144.4 87.4) (end 144.4 87.9) (width 0.254) (layer "F.Cu") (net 6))
 (segment (start 146.7 83.5) (end 147.425 84.225) (width 0.254) (layer "F.Cu") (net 2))
 (segment (start 157.6 82.05) (end 157.6 86.15) (width 0.254) (layer "F.Cu") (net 2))
 (segment (start 150.725 84.775) (end 150.5 85) (width 0.254) (layer "F.Cu") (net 2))
 (segment (start 139 89) (end 154.75 89) (width 0.254) (layer "F.Cu") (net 2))
 (segment (start 141.6 83.5) (end 146.7 83.5) (width 0.254) (layer "F.Cu") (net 2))
 (segment (start 137.85 87.85) (end 139 89) (width 0.254) (layer "F.Cu") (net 2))
 (segment (start 141.6 80) (end 138.9 80) (width 0.254) (layer "F.Cu") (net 2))
 (segment (start 138.95 82.1) (end 141.6 82.1) (width 0.254) (layer "F.Cu") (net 2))
 (segment (start 137.85 82.5) (end 137.85 87.85) (width 0.254) (layer "F.Cu") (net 2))
 (segment (start 150.725 84) (end 151.7 84) (width 0.254) (layer "F.Cu") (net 2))
 (segment (start 138.6 81.75) (end 138.95 82.1) (width 0.254) (layer "F.Cu") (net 2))
 (segment (start 156.65 86.9) (end 156.75 87) (width 0.254) (layer "F.Cu") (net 2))
 (segment (start 156.65 81.1) (end 157.6 82.05) (width 0.254) (layer "F.Cu") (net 2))
 (segment (start 150.5 85) (end 147.825 85) (width 0.254) (layer "F.Cu") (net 2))
 (segment (start 150.725 84) (end 150.725 84.775) (width 0.254) (layer "F.Cu") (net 2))
 (segment (start 154.6 81.1) (end 156.65 81.1) (width 0.254) (layer "F.Cu") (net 2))
 (segment (start 147.825 85) (end 147.425 84.6) (width 0.254) (layer "F.Cu") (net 2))
 (segment (start 154 86.9) (end 156.65 86.9) (width 0.254) (layer "F.Cu") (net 2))
 (segment (start 138.6 80.3) (end 138.6 81.75) (width 0.254) (layer "F.Cu") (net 2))
 (segment (start 138.9 80) (end 138.6 80.3) (width 0.254) (layer "F.Cu") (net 2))
 (segment (start 157.6 86.15) (end 156.75 87) (width 0.254) (layer "F.Cu") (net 2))
 (segment (start 147.425 84.225) (end 147.425 84.6) (width 0.254) (layer "F.Cu") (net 2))
 (segment (start 151.7 84) (end 154.6 81.1) (width 0.254) (layer "F.Cu") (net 2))
 (segment (start 154.75 89) (end 156.75 87) (width 0.254) (layer "F.Cu") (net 2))
 (segment (start 138.6 81.75) (end 137.85 82.5) (width 0.254) (layer "F.Cu") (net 2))
 (via (at 163.35 85.95) (size 0.6) (drill 0.3) (layers "F.Cu" "B.Cu") (free yes) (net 2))
 (via (at 163.35 80.15) (size 0.6) (drill 0.3) (layers "F.Cu" "B.Cu") (free yes) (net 2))
 (segment (start 145.375 86.3) (end 145.925 86.85) (width 0.254) (layer "F.Cu") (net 8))
 (segment (start 141.6 86.3) (end 145.375 86.3) (width 0.254) (layer "F.Cu") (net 8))
 (segment (start 149.175 82) (end 149.125 81.95) (width 0.254) (layer "F.Cu") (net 1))
 (segment (start 149.175 82) (end 149.175 82.95) (width 0.254) (layer "F.Cu") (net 1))
 (segment (start 139 84.9) (end 138.65 84.55) (width 0.254) (layer "F.Cu") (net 1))
 (segment (start 152.45 82.1) (end 152.45 80.55) (width 0.254) (layer "F.Cu") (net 1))
 (segment (start 138.65 84.55) (end 138.65 83.1) (width 0.254) (layer "F.Cu") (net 1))
 (segment (start 154.2 78.8) (end 155.35 78.8) (width 0.254) (layer "F.Cu") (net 1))
 (segment (start 151.6 82.95) (end 152.45 82.1) (width 0.254) (layer "F.Cu") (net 1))
 (segment (start 141.6 84.9) (end 139 84.9) (width 0.254) (layer "F.Cu") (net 1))
 (segment (start 141.6 82.8) (end 146.525 82.8) (width 0.254) (layer "F.Cu") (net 1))
 (segment (start 152.45 80.55) (end 154.2 78.8) (width 0.254) (layer "F.Cu") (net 1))
 (segment (start 141.6 85.6) (end 141.6 84.9) (width 0.254) (layer "F.Cu") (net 1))
 (segment (start 138.95 82.8) (end 141.6 82.8) (width 0.254) (layer "F.Cu") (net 1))
 (segment (start 149.175 84) (end 149.2 84) (width 0.254) (layer "F.Cu") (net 1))
 (segment (start 149.175 82.95) (end 149.175 84) (width 0.254) (layer "F.Cu") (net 1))
 (segment (start 138.65 83.1) (end 138.95 82.8) (width 0.254) (layer "F.Cu") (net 1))
 (segment (start 146.525 82.8) (end 147.375 81.95) (width 0.254) (layer "F.Cu") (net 1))
 (segment (start 149.175 82.95) (end 151.6 82.95) (width 0.254) (layer "F.Cu") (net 1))
 (segment (start 147.375 81.95) (end 149.125 81.95) (width 0.254) (layer "F.Cu") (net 1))
 (segment (start 141.6 81.4) (end 145.175 81.4) (width 0.254) (layer "F.Cu") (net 4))
 (segment (start 145.175 81.4) (end 145.725 81.95) (width 0.254) (layer "F.Cu") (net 4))
 (segment (start 146.65 81.025) (end 145.725 81.95) (width 0.254) (layer "F.Cu") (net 4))
 (segment (start 146.65 79.3) (end 146.65 81.025) (width 0.254) (layer "F.Cu") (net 4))
 (segment (start 141.6 80.7) (end 144.2 80.7) (width 0.254) (layer "F.Cu") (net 5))
 (segment (start 144.2 80.7) (end 144.45 80.45) (width 0.254) (layer "F.Cu") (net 5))
 (segment (start 144.45 80.45) (end 144.45 78.25) (width 0.254) (layer "F.Cu") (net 5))
 (segment (start 148.75 77.5) (end 150.4 79.15) (width 0.254) (layer "F.Cu") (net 5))
 (segment (start 150.775 81.95) (end 150.775 79.525) (width 0.254) (layer "F.Cu") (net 5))
 (segment (start 144.45 78.25) (end 145.2 77.5) (width 0.254) (layer "F.Cu") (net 5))
 (segment (start 150.775 79.525) (end 150.4 79.15) (width 0.254) (layer "F.Cu") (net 5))
 (segment (start 145.2 77.5) (end 148.75 77.5) (width 0.254) (layer "F.Cu") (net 5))
 (segment (start 145.375 84.2) (end 145.775 84.6) (width 0.254) (layer "F.Cu") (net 3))
 (segment (start 141.6 84.2) (end 145.375 84.2) (width 0.254) (layer "F.Cu") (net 3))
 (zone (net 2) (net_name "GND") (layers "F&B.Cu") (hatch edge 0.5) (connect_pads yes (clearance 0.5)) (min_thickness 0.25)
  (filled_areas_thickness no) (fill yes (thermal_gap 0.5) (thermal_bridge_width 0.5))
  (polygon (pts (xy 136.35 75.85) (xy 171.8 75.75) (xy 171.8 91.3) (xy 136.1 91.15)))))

